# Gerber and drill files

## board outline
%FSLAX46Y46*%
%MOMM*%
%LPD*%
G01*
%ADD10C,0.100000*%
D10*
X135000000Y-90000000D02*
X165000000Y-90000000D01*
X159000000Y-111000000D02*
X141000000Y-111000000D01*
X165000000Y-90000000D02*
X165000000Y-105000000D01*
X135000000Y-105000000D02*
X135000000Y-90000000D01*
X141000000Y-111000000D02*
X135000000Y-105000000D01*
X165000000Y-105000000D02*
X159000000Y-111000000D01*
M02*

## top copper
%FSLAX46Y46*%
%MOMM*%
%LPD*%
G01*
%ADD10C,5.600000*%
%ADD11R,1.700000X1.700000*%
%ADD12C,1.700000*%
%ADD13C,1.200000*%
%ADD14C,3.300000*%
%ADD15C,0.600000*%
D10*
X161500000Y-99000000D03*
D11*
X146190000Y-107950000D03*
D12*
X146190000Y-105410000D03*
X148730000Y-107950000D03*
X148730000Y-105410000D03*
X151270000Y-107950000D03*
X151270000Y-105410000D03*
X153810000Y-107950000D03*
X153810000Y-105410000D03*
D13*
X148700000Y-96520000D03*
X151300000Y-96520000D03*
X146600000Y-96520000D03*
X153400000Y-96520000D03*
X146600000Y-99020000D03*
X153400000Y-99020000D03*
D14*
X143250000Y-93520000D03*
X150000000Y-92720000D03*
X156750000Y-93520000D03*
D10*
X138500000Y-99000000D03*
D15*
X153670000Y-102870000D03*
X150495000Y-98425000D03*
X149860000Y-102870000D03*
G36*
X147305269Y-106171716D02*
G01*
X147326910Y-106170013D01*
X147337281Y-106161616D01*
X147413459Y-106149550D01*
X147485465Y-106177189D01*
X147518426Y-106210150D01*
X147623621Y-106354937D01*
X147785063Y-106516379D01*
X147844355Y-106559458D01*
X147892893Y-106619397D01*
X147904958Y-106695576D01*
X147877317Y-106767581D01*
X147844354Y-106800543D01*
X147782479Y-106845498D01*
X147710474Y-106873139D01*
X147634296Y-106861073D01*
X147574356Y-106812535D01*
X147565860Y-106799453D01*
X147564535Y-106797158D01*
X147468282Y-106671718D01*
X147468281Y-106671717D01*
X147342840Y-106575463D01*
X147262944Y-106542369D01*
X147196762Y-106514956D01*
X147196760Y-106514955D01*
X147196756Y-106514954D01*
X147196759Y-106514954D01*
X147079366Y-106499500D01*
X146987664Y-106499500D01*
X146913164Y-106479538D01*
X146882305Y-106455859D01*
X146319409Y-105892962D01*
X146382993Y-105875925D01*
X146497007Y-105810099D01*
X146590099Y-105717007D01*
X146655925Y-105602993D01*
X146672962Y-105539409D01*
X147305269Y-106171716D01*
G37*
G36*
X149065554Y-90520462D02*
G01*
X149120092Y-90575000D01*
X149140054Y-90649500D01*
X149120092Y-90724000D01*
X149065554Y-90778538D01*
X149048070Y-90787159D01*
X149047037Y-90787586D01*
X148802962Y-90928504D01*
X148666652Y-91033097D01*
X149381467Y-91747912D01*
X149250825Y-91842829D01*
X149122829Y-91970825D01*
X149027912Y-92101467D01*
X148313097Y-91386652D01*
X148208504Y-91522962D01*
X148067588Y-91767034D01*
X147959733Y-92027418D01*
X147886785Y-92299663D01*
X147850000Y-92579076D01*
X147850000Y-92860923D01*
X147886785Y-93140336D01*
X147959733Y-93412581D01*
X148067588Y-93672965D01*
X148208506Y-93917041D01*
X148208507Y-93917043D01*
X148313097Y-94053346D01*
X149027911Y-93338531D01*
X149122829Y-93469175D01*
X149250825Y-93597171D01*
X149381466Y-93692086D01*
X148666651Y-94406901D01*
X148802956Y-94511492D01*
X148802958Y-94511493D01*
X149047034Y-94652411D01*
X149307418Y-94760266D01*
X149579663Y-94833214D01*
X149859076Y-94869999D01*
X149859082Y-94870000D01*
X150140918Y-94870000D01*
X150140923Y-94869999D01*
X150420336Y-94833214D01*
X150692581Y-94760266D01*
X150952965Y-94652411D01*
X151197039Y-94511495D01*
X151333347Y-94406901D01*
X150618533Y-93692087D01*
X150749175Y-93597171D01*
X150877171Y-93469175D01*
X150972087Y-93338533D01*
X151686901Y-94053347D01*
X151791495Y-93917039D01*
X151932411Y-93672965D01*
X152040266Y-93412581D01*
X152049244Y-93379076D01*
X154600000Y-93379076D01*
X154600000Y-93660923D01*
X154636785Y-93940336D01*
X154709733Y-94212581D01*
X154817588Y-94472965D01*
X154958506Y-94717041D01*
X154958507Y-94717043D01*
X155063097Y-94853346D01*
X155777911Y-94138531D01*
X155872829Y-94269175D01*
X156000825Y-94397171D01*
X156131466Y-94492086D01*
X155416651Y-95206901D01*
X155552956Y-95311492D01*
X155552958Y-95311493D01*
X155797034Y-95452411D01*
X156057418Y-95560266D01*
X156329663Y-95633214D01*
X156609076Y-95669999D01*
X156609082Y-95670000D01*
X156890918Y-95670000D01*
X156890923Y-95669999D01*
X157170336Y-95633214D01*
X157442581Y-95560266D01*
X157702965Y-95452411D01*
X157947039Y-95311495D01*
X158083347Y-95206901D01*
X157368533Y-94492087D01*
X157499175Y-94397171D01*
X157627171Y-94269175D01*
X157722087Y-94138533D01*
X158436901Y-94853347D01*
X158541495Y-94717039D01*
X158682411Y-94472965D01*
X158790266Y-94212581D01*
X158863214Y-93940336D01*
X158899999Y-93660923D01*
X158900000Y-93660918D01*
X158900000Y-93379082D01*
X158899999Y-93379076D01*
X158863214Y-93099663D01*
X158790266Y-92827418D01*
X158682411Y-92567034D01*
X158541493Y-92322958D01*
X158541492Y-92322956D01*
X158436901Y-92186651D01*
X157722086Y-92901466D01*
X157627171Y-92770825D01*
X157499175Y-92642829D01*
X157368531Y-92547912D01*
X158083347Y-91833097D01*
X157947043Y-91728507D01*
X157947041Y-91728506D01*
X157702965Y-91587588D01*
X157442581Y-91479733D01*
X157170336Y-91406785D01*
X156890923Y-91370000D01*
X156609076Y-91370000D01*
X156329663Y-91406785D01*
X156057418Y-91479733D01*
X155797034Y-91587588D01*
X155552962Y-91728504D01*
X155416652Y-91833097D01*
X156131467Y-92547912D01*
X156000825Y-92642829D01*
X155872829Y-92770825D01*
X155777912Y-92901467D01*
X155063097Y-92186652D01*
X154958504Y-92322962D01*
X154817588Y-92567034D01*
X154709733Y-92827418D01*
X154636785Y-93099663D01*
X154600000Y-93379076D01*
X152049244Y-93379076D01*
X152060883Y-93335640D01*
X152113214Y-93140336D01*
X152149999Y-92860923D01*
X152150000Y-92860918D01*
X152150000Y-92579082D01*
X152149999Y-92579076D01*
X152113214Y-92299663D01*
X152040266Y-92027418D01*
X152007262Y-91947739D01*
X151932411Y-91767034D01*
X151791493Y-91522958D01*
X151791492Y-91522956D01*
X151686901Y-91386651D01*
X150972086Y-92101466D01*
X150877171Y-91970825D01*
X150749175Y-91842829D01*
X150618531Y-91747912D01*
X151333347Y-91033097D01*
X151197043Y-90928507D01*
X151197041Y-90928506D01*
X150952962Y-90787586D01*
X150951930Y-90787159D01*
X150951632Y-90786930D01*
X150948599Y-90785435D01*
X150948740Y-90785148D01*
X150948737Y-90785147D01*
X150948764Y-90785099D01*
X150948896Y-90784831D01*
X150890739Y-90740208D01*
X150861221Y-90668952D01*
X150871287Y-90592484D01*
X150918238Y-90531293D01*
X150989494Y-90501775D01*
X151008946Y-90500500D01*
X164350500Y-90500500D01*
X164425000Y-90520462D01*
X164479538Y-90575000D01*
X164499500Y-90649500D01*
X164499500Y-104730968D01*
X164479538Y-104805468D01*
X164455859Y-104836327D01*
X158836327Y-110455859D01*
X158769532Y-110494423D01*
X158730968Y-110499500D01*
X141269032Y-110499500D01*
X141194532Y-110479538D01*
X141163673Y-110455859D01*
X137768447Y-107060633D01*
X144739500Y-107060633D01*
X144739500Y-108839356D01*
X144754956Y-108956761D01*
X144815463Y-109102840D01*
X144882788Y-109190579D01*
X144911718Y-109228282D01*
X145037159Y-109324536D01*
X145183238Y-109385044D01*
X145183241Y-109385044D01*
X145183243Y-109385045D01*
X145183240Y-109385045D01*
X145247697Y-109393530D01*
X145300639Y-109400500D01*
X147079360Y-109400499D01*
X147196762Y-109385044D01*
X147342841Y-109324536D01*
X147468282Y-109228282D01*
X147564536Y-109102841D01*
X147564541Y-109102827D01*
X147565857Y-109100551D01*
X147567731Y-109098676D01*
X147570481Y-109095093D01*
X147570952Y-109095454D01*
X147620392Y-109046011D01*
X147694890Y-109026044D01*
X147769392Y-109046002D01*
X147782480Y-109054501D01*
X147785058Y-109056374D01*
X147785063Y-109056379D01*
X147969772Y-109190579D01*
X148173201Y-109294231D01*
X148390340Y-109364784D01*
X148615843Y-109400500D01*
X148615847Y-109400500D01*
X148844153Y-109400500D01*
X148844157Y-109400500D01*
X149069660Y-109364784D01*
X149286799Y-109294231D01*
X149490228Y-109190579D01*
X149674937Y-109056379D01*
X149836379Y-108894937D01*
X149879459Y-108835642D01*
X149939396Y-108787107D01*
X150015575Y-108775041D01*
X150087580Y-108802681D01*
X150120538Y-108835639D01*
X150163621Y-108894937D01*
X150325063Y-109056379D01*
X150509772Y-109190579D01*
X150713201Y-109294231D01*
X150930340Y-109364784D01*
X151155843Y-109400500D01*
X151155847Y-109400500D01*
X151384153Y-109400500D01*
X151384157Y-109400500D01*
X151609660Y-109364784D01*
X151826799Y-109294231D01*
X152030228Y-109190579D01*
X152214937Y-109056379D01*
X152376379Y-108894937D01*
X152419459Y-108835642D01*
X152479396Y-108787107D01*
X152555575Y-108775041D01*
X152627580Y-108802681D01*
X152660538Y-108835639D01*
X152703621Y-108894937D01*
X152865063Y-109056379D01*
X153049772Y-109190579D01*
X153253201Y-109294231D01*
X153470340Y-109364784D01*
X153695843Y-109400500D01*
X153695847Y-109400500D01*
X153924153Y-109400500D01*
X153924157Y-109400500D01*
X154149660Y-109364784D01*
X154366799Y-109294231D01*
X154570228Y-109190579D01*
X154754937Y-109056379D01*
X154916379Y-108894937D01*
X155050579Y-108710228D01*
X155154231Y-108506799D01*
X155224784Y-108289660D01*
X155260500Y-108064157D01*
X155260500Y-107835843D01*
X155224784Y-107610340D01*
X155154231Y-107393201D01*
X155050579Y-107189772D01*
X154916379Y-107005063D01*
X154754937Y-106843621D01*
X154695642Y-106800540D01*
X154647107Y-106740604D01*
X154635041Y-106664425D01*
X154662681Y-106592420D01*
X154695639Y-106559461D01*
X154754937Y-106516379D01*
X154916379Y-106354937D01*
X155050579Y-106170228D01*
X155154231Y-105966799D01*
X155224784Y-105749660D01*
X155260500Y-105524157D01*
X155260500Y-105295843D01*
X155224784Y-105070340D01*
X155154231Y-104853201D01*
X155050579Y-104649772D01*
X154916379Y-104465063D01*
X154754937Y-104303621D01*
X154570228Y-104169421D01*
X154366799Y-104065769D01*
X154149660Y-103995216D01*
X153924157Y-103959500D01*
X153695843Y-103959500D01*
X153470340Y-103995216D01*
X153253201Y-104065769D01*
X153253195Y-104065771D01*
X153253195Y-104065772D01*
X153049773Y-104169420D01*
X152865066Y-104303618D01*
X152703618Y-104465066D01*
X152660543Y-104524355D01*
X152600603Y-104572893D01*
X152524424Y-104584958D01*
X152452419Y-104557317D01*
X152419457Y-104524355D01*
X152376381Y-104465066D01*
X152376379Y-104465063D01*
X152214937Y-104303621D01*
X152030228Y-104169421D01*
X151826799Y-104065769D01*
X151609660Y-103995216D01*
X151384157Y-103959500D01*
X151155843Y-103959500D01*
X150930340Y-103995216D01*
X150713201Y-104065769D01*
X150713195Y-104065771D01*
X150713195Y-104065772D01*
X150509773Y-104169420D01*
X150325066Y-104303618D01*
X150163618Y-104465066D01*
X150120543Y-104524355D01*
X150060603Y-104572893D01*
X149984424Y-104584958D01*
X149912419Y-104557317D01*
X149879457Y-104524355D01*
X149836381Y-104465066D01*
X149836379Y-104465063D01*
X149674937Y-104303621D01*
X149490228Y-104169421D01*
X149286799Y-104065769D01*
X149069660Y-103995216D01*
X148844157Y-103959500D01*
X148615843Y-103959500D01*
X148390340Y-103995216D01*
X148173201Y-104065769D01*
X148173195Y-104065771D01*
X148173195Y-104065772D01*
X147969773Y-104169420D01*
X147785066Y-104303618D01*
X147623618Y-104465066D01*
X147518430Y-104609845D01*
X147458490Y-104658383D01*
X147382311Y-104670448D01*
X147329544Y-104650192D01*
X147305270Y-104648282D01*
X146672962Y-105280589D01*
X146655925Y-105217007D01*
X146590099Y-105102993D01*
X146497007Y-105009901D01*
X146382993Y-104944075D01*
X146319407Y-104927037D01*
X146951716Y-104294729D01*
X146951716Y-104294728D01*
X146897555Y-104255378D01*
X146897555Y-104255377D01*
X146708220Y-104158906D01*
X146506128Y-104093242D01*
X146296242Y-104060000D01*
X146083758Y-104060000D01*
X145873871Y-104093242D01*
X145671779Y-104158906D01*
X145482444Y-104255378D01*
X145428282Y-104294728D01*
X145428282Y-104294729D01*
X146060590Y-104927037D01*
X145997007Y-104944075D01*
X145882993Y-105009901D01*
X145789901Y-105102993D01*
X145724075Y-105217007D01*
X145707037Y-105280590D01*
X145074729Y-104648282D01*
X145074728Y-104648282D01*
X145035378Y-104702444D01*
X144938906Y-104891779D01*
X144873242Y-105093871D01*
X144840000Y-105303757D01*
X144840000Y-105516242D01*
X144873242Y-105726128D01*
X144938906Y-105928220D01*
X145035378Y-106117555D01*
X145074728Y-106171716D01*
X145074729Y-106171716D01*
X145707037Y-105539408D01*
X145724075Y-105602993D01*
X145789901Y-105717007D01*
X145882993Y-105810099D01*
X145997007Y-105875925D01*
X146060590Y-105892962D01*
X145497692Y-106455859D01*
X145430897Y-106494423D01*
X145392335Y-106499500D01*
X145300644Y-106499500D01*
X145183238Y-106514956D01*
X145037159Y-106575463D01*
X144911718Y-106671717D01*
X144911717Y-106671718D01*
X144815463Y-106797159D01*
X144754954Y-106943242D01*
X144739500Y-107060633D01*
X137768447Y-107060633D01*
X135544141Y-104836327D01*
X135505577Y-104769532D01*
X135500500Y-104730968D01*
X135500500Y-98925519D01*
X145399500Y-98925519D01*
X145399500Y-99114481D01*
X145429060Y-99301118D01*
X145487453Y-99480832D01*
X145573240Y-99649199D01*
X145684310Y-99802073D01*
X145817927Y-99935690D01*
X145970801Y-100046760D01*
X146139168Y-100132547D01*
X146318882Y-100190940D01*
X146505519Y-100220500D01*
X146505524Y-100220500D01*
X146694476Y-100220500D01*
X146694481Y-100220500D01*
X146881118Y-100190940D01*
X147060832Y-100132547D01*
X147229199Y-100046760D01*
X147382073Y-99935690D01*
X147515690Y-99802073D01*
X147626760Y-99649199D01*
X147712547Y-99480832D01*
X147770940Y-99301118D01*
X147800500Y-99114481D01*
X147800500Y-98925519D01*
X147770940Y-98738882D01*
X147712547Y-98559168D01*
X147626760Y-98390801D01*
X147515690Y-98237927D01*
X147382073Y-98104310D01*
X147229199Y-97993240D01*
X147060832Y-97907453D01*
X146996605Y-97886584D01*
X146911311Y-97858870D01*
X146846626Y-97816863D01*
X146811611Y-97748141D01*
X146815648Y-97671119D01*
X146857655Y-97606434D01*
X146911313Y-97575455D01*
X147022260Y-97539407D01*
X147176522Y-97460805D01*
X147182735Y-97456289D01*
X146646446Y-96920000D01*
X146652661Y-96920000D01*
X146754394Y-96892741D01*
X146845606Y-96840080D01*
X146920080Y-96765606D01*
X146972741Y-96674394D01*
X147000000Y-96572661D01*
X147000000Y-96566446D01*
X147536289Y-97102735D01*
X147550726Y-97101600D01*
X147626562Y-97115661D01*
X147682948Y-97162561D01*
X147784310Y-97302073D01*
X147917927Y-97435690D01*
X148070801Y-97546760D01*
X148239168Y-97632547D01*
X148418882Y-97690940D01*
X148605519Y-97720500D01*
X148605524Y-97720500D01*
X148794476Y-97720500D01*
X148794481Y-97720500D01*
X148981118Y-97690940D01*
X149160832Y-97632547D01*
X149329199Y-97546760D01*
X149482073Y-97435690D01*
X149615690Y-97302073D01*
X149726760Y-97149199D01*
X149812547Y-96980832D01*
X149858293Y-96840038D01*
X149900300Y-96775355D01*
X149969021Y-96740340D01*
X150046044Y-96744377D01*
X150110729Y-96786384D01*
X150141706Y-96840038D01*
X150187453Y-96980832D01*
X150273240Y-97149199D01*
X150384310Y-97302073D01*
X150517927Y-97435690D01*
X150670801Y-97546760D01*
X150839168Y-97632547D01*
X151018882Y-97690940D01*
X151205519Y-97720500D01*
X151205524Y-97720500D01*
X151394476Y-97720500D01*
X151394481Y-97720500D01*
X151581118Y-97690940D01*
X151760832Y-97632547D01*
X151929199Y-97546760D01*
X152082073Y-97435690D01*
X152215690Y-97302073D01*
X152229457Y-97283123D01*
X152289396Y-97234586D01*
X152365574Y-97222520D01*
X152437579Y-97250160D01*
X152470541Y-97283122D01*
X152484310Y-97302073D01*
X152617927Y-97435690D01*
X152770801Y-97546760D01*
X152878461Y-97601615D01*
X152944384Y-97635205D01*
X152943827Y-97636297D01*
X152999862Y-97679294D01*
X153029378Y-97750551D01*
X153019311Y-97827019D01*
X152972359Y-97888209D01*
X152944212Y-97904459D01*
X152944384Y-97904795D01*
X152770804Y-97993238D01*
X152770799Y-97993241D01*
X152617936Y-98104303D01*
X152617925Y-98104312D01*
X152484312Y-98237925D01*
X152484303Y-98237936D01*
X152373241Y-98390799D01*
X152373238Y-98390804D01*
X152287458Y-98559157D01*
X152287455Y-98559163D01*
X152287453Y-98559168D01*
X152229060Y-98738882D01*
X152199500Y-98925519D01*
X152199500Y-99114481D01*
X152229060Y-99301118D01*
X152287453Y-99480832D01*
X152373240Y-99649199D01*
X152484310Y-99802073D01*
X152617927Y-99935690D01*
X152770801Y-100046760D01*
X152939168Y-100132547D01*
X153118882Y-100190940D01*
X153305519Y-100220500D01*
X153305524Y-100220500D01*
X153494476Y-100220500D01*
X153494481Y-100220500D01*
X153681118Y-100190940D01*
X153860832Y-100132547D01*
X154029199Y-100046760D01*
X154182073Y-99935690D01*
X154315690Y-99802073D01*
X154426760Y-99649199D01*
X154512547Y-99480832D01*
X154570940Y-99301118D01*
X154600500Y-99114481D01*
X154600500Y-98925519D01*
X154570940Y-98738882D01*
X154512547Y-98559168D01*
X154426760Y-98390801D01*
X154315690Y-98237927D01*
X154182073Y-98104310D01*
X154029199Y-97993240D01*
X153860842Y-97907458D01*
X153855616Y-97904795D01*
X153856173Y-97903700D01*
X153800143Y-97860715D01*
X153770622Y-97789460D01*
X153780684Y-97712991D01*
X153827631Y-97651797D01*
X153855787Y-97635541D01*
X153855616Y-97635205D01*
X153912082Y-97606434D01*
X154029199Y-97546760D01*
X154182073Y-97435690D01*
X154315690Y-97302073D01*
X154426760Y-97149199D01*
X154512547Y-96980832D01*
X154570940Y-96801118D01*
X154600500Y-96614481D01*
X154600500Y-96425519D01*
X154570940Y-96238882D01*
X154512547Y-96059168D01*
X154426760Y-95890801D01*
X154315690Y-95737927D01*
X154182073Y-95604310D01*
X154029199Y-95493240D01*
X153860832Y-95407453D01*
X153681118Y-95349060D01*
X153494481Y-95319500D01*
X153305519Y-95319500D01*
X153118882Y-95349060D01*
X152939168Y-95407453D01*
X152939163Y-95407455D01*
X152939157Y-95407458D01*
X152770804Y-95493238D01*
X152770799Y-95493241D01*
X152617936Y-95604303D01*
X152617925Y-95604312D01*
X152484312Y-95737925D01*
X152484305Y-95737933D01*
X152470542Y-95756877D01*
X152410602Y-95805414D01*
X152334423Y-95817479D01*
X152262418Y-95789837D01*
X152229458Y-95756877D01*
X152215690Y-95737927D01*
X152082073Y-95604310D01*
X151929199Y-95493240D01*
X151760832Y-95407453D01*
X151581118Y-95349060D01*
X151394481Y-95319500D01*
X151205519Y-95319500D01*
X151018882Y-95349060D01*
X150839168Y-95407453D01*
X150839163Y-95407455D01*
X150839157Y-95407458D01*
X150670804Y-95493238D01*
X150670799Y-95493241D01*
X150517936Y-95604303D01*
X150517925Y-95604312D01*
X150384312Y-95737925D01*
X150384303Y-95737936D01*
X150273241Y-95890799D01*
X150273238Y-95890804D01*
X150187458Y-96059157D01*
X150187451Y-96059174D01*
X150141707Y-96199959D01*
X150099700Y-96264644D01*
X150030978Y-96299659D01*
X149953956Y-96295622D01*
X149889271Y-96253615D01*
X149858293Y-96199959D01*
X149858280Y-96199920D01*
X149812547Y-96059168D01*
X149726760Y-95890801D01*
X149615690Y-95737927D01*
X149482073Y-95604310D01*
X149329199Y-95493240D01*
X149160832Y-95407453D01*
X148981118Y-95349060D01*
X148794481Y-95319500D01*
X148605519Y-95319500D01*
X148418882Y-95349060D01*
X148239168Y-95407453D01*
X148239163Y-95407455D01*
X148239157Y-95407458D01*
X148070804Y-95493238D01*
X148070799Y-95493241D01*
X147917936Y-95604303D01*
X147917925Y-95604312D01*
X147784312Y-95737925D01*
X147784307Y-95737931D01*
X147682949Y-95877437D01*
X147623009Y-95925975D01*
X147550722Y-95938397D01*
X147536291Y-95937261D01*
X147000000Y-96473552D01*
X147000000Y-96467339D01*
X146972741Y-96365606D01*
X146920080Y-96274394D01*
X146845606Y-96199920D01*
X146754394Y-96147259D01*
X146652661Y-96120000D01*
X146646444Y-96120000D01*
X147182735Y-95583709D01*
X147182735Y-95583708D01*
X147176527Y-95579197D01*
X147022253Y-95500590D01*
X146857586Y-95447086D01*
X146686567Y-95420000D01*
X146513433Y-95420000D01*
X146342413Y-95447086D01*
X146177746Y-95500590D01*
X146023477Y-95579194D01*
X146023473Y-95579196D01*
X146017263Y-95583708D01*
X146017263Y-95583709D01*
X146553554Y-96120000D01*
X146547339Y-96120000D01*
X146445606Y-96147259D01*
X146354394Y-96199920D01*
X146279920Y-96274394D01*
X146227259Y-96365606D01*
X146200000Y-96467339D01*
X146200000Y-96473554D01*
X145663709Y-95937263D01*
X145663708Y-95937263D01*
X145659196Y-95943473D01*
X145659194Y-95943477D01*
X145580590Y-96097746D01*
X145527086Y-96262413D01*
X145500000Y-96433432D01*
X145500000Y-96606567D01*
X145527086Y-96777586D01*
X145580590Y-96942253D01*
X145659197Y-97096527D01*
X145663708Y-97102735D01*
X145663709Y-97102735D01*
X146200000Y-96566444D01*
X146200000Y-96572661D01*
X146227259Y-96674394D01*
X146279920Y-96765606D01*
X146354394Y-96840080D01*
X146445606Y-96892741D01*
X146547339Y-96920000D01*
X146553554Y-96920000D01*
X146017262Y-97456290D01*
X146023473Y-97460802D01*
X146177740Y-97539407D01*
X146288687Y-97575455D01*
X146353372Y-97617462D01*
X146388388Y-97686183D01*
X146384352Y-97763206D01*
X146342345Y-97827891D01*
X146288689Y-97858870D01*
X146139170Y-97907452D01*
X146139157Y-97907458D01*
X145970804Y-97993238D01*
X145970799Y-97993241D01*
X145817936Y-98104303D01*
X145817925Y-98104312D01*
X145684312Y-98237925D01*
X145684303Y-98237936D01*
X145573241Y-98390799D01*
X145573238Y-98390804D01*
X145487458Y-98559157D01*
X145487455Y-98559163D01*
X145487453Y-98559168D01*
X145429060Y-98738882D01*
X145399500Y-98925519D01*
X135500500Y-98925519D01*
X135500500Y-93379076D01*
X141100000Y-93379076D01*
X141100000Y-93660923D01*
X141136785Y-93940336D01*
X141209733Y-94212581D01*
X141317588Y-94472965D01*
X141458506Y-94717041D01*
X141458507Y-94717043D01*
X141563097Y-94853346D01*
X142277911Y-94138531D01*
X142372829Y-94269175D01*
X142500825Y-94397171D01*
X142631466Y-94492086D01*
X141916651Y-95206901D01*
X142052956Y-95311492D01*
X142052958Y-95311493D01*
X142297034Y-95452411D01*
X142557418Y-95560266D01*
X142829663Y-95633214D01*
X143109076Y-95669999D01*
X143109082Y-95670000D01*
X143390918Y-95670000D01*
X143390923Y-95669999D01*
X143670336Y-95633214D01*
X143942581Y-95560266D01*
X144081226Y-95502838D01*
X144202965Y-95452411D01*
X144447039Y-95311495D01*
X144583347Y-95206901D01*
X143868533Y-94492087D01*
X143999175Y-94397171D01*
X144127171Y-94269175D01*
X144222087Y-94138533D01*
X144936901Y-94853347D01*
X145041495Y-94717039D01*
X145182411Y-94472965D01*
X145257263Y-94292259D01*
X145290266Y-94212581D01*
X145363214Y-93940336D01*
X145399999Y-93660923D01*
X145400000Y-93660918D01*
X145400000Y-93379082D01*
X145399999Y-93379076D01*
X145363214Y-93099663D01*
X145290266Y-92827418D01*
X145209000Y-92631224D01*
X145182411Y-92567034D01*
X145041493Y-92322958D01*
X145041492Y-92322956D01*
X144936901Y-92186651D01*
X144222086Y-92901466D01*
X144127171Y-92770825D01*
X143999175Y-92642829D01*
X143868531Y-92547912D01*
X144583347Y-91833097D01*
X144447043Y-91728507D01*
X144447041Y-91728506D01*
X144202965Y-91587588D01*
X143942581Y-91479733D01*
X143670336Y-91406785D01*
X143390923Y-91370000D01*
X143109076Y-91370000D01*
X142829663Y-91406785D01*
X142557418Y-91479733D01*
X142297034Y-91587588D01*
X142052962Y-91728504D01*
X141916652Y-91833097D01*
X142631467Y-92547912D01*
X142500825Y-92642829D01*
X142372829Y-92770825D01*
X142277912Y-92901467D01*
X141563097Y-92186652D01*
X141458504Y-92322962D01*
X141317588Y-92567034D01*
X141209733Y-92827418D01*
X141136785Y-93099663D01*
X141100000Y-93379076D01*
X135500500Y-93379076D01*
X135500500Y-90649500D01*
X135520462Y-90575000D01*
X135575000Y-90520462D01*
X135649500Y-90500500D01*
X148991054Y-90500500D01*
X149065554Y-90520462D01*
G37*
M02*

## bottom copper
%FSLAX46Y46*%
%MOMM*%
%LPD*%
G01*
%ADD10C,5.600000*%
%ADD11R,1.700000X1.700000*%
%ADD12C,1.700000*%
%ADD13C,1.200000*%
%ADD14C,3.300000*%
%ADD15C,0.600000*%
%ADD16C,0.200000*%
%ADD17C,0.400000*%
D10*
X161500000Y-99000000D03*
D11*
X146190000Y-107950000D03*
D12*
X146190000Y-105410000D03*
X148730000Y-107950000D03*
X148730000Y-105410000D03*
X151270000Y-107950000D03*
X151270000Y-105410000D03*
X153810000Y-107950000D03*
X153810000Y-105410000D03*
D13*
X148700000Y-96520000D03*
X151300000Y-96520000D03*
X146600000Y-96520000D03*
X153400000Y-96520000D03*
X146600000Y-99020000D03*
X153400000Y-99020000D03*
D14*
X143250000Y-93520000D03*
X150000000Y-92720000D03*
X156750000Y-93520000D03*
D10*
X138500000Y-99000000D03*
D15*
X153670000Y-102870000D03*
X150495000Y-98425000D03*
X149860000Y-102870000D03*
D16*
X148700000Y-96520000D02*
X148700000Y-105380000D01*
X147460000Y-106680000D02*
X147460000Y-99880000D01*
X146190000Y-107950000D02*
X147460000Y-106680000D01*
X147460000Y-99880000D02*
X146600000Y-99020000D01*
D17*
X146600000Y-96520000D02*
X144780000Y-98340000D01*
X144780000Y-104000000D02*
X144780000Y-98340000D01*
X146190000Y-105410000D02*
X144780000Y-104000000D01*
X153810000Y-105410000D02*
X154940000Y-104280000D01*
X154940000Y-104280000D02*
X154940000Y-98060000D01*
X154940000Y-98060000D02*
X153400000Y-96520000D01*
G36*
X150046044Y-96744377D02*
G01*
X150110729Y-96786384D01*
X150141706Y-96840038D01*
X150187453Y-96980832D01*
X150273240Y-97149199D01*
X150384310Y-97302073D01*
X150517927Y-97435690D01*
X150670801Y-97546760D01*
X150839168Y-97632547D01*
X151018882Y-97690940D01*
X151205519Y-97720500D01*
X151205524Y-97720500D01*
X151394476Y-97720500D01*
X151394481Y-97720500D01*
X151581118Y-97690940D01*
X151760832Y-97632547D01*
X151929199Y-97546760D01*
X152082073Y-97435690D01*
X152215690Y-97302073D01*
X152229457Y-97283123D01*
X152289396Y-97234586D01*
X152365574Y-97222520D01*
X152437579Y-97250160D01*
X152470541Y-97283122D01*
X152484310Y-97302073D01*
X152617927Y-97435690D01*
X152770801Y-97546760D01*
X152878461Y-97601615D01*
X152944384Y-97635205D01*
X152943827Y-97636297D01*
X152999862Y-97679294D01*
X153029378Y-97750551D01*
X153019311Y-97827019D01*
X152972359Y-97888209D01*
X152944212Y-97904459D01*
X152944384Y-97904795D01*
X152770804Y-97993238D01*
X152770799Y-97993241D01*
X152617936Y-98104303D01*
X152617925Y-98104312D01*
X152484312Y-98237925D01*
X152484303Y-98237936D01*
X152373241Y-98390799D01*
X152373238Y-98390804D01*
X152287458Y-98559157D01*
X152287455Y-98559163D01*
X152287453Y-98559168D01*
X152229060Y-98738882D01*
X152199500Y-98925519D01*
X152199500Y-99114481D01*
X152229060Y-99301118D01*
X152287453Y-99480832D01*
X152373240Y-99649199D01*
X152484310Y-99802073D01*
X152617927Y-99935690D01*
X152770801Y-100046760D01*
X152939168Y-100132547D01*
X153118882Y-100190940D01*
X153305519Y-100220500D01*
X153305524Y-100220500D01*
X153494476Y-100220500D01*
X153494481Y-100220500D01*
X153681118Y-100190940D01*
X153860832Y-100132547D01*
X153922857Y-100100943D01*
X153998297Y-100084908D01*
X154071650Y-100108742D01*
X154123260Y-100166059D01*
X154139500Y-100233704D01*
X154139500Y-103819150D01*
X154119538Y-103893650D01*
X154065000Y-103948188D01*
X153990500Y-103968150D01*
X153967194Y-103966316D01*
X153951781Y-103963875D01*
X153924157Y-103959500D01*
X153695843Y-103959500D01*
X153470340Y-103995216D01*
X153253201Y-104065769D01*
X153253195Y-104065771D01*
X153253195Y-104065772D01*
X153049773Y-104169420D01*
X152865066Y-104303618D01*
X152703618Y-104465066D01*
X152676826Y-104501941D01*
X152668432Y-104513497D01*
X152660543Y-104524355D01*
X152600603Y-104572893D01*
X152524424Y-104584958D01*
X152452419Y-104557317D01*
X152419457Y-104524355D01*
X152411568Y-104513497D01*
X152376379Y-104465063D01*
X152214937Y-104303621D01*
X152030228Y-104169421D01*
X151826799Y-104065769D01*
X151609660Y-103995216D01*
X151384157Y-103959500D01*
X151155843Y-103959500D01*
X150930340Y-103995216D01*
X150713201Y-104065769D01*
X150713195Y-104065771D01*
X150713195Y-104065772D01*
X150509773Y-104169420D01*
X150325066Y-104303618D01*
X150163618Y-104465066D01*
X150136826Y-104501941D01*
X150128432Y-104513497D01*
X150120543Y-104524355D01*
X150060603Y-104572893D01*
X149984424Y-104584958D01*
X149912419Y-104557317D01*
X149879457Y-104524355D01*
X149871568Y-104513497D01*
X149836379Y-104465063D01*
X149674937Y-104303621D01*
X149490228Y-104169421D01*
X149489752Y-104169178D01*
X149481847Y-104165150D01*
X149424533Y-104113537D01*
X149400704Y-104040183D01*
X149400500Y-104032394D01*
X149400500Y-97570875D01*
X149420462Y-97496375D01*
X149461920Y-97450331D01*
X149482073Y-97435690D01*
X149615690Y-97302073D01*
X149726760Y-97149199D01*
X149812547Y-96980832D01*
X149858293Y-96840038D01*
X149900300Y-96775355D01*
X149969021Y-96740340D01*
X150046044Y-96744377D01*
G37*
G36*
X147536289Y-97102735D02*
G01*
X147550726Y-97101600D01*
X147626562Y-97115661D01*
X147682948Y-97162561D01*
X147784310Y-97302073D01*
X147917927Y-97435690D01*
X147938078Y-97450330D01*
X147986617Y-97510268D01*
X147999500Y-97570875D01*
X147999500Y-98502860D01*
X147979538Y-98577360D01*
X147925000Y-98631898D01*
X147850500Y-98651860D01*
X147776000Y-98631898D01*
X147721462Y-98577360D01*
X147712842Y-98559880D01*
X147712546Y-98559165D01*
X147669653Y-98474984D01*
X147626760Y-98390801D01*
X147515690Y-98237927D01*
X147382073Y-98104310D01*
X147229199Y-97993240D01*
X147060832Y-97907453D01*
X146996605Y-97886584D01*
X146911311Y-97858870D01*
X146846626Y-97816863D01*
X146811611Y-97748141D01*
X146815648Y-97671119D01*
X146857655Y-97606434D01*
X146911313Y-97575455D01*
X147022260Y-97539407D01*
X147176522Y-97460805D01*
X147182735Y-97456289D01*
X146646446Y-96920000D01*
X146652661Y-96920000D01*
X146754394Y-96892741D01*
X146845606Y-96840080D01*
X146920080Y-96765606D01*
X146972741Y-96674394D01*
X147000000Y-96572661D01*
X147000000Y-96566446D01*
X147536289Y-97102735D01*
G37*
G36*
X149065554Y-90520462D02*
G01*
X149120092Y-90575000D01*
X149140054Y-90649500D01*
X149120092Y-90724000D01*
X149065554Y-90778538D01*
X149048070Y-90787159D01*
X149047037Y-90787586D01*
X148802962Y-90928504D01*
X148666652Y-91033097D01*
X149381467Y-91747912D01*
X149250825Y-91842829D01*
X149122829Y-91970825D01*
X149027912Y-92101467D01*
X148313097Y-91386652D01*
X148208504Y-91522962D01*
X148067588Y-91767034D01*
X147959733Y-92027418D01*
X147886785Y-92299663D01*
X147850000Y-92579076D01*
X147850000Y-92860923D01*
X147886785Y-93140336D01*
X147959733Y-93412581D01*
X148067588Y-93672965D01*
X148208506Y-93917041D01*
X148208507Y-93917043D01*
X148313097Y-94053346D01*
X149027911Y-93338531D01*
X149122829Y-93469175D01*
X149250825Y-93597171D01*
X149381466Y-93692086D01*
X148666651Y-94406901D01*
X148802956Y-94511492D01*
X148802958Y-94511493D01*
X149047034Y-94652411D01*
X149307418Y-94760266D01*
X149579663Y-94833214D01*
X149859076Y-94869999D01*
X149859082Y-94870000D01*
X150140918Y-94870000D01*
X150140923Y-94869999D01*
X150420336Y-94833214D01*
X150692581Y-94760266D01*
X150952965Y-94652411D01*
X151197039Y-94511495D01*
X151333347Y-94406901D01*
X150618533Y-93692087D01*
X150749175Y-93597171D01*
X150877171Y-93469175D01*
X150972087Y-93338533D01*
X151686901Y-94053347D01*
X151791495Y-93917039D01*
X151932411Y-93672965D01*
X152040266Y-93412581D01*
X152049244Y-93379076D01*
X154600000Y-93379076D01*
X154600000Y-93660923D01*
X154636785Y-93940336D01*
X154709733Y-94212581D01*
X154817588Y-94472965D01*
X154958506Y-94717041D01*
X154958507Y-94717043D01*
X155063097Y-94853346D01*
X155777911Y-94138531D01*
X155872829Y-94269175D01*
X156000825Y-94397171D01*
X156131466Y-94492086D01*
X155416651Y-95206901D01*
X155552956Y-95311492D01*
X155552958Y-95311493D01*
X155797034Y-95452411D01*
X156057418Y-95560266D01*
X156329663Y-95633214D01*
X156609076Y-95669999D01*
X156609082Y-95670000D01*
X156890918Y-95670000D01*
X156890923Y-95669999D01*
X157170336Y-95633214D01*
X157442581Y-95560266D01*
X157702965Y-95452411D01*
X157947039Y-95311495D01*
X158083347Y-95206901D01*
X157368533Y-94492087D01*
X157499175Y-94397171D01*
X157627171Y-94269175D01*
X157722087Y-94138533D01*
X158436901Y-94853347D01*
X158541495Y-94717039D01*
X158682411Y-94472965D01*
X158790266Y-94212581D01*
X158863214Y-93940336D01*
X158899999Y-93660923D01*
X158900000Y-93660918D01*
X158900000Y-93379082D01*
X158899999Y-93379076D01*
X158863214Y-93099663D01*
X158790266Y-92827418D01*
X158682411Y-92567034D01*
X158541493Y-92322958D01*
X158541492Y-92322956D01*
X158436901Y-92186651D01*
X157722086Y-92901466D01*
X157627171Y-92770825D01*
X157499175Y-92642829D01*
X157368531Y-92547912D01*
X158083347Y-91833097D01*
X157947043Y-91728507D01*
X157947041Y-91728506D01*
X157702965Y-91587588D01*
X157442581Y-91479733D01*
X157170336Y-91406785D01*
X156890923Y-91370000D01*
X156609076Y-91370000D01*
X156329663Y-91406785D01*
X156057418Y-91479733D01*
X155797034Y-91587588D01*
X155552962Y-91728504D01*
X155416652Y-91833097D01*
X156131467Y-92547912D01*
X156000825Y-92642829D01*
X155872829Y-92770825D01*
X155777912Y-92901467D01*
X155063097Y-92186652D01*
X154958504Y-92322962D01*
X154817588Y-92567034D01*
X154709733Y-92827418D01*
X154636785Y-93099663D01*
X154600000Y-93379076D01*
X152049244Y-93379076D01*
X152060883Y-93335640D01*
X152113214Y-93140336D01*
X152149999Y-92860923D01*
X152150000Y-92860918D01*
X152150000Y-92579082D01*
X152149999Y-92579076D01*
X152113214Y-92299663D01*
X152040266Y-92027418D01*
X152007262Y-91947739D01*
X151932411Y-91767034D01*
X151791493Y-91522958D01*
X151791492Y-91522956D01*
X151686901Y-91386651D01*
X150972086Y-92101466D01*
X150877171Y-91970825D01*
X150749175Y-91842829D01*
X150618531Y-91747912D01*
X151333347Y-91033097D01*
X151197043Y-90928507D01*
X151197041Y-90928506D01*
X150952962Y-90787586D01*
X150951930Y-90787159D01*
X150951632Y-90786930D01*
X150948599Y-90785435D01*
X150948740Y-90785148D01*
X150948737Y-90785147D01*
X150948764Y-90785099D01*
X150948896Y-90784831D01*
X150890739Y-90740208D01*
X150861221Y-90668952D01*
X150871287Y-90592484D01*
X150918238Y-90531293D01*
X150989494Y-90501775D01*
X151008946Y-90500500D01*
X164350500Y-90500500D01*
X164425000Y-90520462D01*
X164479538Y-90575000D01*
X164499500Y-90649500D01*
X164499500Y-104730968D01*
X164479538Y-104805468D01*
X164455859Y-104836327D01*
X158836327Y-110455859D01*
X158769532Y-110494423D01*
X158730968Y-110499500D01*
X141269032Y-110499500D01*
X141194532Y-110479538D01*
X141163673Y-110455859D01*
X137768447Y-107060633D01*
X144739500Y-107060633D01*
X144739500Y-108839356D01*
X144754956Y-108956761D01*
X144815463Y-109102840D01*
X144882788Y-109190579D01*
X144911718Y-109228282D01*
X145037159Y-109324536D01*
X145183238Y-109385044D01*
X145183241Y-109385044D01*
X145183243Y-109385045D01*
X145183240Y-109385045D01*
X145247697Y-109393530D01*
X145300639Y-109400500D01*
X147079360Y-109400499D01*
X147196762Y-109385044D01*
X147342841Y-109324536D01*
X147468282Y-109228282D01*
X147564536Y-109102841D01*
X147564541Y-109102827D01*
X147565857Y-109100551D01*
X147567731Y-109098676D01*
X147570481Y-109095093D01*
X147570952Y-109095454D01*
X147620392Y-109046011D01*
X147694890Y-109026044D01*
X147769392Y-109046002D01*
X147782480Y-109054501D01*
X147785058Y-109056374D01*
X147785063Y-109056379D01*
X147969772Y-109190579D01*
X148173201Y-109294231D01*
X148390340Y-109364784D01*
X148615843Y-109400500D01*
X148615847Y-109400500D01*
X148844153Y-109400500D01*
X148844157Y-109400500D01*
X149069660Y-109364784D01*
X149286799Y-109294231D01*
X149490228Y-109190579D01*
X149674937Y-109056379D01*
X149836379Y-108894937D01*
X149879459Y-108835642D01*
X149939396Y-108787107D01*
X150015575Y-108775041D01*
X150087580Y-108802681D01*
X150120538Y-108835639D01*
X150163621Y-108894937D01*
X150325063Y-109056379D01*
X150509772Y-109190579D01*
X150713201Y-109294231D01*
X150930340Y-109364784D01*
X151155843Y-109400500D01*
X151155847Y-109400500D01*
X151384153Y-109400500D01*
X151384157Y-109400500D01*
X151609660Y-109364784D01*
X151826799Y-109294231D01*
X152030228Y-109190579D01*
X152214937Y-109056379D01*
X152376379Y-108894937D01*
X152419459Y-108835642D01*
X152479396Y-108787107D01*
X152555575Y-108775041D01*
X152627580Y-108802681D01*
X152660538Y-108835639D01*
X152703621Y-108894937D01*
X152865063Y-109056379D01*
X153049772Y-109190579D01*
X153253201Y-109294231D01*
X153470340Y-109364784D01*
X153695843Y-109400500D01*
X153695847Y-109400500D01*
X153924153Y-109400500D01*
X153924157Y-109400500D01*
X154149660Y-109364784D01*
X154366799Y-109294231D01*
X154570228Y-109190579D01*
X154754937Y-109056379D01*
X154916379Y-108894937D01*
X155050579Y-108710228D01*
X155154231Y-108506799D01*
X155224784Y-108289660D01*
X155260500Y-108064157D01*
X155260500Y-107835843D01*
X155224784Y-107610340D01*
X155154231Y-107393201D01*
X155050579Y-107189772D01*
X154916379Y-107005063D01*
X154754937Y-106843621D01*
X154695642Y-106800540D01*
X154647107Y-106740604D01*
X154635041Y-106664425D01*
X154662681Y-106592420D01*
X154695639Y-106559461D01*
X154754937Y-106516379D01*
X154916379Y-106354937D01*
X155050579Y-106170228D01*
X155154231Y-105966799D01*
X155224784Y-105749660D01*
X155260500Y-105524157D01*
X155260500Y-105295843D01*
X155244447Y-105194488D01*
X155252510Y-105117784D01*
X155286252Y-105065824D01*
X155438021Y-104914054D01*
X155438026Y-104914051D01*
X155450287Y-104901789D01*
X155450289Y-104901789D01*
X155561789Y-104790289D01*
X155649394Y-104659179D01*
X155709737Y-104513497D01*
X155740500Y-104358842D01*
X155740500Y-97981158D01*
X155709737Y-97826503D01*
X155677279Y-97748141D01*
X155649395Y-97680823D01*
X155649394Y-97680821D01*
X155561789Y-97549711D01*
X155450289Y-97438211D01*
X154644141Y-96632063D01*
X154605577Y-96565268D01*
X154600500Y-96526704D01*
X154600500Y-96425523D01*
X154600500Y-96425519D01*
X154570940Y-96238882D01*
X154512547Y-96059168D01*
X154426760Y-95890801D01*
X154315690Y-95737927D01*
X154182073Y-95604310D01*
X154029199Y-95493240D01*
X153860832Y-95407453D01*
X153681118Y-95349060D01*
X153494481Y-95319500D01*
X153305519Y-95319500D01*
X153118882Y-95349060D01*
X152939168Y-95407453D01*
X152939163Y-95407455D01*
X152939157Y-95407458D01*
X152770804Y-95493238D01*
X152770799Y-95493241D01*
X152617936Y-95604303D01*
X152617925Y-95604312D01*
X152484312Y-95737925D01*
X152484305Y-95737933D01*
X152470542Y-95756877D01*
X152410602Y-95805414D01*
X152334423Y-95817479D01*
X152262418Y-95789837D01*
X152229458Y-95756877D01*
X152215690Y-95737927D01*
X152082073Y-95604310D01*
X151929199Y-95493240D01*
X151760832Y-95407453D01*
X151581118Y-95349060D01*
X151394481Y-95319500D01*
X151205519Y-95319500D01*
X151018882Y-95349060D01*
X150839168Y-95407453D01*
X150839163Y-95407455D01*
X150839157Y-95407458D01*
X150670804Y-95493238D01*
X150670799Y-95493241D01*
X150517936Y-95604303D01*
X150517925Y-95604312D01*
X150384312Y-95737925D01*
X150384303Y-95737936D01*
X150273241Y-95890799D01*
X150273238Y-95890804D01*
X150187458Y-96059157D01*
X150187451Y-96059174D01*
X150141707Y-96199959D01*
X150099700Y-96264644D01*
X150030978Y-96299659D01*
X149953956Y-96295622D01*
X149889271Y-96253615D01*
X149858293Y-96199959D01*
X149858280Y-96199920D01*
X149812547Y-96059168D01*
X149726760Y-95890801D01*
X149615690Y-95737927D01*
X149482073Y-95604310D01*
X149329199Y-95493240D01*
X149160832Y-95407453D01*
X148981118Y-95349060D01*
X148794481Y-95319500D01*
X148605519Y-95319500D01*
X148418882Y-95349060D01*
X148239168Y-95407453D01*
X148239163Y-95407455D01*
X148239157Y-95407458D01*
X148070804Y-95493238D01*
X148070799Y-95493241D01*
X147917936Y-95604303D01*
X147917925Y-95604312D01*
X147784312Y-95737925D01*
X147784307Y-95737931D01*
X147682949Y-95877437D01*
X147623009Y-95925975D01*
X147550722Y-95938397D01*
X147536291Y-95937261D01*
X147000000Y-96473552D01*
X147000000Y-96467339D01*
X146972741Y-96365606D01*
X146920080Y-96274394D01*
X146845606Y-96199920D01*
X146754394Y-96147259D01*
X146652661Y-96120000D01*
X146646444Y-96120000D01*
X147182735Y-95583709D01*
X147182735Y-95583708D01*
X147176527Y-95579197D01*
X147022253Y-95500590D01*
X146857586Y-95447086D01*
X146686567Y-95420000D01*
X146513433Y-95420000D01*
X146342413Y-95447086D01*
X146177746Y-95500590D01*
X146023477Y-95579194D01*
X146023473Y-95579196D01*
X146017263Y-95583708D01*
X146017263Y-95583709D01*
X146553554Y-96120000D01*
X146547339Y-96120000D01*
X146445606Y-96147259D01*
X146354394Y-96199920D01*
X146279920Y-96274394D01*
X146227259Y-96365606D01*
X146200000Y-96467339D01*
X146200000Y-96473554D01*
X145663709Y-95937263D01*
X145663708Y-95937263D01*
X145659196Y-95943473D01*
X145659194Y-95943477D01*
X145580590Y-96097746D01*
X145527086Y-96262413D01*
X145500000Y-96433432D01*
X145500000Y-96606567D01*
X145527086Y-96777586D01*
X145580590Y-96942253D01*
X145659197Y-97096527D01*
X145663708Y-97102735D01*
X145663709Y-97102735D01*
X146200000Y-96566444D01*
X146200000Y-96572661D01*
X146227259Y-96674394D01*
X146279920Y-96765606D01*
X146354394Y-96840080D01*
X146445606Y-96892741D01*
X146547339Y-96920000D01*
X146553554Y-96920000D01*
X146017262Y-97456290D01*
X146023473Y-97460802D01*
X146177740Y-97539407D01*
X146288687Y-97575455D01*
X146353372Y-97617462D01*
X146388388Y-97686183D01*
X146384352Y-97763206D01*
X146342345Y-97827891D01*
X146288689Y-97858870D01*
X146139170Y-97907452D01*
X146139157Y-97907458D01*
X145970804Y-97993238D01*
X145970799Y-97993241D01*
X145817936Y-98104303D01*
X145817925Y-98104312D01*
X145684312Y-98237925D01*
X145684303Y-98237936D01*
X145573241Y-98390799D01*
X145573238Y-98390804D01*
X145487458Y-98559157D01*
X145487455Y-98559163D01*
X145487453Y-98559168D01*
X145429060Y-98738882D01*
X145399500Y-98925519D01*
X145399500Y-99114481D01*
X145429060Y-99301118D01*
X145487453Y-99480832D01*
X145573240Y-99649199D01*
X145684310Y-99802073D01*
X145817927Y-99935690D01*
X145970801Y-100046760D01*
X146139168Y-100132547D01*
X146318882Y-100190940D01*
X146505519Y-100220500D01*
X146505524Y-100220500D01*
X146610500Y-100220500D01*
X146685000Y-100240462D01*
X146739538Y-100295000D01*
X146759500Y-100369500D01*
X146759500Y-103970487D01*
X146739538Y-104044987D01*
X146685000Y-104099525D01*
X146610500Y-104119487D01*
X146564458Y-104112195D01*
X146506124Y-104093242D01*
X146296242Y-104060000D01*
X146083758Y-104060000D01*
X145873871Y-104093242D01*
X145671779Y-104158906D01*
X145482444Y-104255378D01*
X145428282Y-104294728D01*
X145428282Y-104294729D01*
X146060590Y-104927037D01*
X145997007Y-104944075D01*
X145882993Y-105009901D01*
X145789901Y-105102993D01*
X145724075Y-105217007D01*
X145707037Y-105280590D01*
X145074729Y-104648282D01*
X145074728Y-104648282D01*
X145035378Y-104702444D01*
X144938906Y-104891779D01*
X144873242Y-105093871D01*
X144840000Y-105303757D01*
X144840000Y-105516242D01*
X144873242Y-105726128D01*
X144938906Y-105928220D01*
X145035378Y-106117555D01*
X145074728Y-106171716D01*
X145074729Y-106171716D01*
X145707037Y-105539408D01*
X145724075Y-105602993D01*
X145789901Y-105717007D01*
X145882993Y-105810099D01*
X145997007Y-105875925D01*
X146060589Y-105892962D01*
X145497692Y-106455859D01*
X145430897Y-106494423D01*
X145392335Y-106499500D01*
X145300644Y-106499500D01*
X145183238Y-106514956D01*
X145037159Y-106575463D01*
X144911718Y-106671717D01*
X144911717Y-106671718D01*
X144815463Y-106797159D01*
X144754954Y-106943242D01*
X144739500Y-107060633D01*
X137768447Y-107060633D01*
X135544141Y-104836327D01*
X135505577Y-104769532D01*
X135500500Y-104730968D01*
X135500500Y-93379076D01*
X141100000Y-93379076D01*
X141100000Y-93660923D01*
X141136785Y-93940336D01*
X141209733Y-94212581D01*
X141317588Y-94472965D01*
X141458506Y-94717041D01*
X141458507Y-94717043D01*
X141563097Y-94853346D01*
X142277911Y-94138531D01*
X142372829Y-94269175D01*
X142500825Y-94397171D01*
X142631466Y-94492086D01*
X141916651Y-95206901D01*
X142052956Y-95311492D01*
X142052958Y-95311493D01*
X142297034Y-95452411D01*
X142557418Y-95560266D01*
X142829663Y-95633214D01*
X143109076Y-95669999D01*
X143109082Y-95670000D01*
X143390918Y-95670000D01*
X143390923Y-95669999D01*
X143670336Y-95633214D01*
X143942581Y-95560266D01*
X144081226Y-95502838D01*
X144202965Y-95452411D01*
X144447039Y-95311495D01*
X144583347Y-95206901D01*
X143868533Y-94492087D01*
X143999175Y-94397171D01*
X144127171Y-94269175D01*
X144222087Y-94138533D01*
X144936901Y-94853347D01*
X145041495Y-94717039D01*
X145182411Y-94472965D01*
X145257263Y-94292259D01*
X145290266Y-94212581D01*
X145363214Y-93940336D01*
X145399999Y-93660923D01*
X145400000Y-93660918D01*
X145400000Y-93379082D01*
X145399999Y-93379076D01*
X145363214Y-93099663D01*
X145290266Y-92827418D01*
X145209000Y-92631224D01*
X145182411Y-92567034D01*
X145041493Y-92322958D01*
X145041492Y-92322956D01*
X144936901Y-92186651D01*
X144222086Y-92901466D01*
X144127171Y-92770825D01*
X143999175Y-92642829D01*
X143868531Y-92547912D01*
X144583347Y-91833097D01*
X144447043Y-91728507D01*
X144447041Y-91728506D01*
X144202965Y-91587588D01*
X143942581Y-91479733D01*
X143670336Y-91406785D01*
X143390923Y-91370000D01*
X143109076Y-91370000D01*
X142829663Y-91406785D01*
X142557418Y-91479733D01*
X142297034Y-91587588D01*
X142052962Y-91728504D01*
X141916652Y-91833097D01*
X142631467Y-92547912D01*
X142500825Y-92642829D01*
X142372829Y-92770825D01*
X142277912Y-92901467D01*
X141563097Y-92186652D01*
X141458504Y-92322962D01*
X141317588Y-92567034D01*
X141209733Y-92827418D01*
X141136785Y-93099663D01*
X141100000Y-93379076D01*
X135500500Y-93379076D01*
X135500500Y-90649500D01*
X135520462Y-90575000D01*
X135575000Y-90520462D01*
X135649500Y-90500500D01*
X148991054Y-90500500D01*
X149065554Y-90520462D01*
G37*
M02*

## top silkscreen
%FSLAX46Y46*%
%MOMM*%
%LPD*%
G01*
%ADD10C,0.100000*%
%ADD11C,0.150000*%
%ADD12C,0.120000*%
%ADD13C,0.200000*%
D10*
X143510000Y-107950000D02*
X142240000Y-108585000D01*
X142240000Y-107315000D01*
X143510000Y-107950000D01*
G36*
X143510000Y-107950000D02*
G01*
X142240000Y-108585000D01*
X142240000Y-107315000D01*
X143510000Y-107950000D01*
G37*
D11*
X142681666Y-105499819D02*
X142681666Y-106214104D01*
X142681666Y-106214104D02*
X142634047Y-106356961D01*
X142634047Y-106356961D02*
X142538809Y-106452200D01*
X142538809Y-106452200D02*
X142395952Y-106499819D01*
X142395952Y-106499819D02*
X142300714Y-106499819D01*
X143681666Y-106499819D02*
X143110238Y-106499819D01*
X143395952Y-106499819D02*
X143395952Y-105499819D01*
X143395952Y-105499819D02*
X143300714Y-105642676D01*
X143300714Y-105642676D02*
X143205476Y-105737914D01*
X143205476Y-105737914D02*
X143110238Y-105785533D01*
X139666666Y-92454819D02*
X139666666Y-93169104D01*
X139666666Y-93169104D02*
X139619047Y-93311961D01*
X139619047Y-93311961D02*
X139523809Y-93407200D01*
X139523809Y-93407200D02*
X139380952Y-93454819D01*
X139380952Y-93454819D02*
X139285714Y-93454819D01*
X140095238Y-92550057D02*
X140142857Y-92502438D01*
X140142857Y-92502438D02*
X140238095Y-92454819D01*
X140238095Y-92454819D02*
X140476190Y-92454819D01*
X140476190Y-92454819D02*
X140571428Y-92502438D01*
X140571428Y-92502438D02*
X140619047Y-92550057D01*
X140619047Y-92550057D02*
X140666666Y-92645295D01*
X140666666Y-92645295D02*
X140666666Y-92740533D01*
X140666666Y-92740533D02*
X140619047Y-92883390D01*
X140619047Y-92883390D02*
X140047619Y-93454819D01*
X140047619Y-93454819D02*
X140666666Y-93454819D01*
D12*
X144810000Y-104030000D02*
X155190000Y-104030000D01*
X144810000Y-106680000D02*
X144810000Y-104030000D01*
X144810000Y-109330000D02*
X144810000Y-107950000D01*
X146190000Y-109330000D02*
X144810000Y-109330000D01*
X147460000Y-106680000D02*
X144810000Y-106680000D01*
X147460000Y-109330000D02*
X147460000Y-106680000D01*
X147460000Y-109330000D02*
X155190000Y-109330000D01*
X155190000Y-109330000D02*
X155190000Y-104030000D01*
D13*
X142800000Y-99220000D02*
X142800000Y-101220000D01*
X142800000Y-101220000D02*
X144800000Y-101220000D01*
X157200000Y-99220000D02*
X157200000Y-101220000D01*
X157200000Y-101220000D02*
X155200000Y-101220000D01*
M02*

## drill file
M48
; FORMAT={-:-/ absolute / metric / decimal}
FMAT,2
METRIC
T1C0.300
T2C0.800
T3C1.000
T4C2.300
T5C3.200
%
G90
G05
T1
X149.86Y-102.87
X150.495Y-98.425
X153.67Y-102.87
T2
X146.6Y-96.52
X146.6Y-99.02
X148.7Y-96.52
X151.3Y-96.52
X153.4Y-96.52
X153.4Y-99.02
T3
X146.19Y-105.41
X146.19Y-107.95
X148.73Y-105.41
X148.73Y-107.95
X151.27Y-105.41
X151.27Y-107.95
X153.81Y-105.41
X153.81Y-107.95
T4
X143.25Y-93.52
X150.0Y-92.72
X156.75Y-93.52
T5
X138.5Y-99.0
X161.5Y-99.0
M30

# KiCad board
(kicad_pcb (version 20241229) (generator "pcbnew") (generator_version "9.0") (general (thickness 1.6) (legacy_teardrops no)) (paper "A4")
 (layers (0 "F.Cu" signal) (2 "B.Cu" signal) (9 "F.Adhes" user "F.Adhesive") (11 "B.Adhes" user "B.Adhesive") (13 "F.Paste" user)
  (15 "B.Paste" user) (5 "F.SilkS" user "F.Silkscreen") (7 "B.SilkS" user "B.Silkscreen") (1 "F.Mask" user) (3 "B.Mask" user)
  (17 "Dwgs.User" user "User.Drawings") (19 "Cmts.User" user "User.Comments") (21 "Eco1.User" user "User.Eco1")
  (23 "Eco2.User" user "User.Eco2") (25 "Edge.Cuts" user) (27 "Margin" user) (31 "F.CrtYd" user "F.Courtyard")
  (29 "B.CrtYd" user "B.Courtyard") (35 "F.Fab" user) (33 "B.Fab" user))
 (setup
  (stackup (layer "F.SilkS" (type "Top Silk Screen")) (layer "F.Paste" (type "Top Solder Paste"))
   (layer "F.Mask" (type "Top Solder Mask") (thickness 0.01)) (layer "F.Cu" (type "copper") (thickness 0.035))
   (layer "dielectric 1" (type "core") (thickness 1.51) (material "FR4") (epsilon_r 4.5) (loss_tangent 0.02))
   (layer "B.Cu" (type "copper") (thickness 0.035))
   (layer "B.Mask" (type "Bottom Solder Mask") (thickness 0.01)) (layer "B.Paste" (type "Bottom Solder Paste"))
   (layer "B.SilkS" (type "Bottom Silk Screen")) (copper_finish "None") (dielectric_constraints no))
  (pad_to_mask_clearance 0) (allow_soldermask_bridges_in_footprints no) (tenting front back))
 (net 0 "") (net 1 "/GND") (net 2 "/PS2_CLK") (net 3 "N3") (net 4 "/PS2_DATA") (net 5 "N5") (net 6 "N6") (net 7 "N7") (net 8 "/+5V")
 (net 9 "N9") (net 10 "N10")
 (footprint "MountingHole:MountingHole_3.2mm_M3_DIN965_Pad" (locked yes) (layer "F.Cu") (at 161.5 99)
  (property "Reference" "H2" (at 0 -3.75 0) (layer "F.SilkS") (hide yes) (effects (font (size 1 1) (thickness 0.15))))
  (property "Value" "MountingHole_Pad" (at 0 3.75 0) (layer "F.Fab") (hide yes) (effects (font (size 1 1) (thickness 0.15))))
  (pad "1" thru_hole circle (at 0 0) (size 5.6 5.6) (drill 3.2) (layers "*.Cu" "*.Mask") (remove_unused_layers no) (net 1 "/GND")
   (zone_connect 2)))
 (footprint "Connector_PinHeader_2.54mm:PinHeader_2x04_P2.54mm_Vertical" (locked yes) (layer "F.Cu") (at 146.19 107.95 90)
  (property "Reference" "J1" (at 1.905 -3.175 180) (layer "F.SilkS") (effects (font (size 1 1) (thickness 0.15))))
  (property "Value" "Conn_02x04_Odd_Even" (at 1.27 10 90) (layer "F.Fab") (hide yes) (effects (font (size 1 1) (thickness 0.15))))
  (fp_line (start 3.92 -1.38) (end 3.92 9) (stroke (width 0.12) (type solid)) (layer "F.SilkS"))
  (fp_line (start 1.27 -1.38) (end 3.92 -1.38) (stroke (width 0.12) (type solid)) (layer "F.SilkS"))
  (fp_line (start -1.38 -1.38) (end 0 -1.38) (stroke (width 0.12) (type solid)) (layer "F.SilkS"))
  (fp_line (start -1.38 0) (end -1.38 -1.38) (stroke (width 0.12) (type solid)) (layer "F.SilkS"))
  (fp_line (start 1.27 1.27) (end 1.27 -1.38) (stroke (width 0.12) (type solid)) (layer "F.SilkS"))
  (fp_line (start -1.38 1.27) (end 1.27 1.27) (stroke (width 0.12) (type solid)) (layer "F.SilkS"))
  (fp_line (start -1.38 1.27) (end -1.38 9) (stroke (width 0.12) (type solid)) (layer "F.SilkS"))
  (fp_line (start -1.38 9) (end 3.92 9) (stroke (width 0.12) (type solid)) (layer "F.SilkS"))
  (pad "1" thru_hole rect (at 0 0 90) (size 1.7 1.7) (drill 1) (layers "*.Cu" "*.Mask") (remove_unused_layers no) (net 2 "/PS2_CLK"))
  (pad "2" thru_hole circle (at 2.54 0 90) (size 1.7 1.7) (drill 1) (layers "*.Cu" "*.Mask") (remove_unused_layers no) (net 1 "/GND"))
  (pad "3" thru_hole circle (at 0 2.54 90) (size 1.7 1.7) (drill 1) (layers "*.Cu" "*.Mask") (remove_unused_layers no) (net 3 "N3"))
  (pad "4" thru_hole circle (at 2.54 2.54 90) (size 1.7 1.7) (drill 1) (layers "*.Cu" "*.Mask") (remove_unused_layers no)
   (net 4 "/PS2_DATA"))
  (pad "5" thru_hole circle (at 0 5.08 90) (size 1.7 1.7) (drill 1) (layers "*.Cu" "*.Mask") (remove_unused_layers no) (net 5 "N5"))
  (pad "6" thru_hole circle (at 2.54 5.08 90) (size 1.7 1.7) (drill 1) (layers "*.Cu" "*.Mask") (remove_unused_layers no) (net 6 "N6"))
  (pad "7" thru_hole circle (at 0 7.62 90) (size 1.7 1.7) (drill 1) (layers "*.Cu" "*.Mask") (remove_unused_layers no) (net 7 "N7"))
  (pad "8" thru_hole circle (at 2.54 7.62 90) (size 1.7 1.7) (drill 1) (layers "*.Cu" "*.Mask") (remove_unused_layers no) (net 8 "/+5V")))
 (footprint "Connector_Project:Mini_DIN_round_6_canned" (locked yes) (layer "F.Cu") (at 150 88.02)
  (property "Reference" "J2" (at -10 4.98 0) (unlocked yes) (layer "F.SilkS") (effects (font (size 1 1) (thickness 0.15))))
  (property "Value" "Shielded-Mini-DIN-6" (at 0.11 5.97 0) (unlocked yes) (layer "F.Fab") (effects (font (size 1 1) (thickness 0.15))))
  (fp_line (start -7.2 11.2) (end -7.2 13.2) (stroke (width 0.2) (type solid)) (layer "F.SilkS"))
  (fp_line (start -7.2 13.2) (end -5.2 13.2) (stroke (width 0.2) (type solid)) (layer "F.SilkS"))
  (fp_line (start 7.2 11.2) (end 7.2 13.2) (stroke (width 0.2) (type solid)) (layer "F.SilkS"))
  (fp_line (start 7.2 13.2) (end 5.2 13.2) (stroke (width 0.2) (type solid)) (layer "F.SilkS"))
  (pad "1" thru_hole circle (at -1.3 8.5 90) (size 1.2 1.2) (drill 0.8) (layers "*.Cu" "*.Mask") (remove_unused_layers no)
   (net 4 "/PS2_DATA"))
  (pad "2" thru_hole circle (at 1.3 8.5 90) (size 1.2 1.2) (drill 0.8) (layers "*.Cu" "*.Mask") (remove_unused_layers no) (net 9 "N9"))
  (pad "3" thru_hole circle (at -3.4 8.5 90) (size 1.2 1.2) (drill 0.8) (layers "*.Cu" "*.Mask") (remove_unused_layers no) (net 1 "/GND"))
  (pad "4" thru_hole circle (at 3.4 8.5 90) (size 1.2 1.2) (drill 0.8) (layers "*.Cu" "*.Mask") (remove_unused_layers no) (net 8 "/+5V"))
  (pad "5" thru_hole circle (at -3.4 11 90) (size 1.2 1.2) (drill 0.8) (layers "*.Cu" "*.Mask") (remove_unused_layers no) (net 2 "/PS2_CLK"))
  (pad "6" thru_hole circle (at 3.4 11 90) (size 1.2 1.2) (drill 0.8) (layers "*.Cu" "*.Mask") (remove_unused_layers no) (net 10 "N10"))
  (pad "SH" thru_hole circle (at -6.75 5.5) (size 3.3 3.3) (drill 2.3) (layers "*.Cu" "*.Mask") (remove_unused_layers no) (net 1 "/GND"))
  (pad "SH" thru_hole circle (at 0 4.7) (size 3.3 3.3) (drill 2.3) (layers "*.Cu" "*.Mask") (remove_unused_layers no) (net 1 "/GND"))
  (pad "SH" thru_hole circle (at 6.75 5.5) (size 3.3 3.3) (drill 2.3) (layers "*.Cu" "*.Mask") (remove_unused_layers no) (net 1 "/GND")))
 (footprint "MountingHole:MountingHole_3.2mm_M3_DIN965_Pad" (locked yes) (layer "F.Cu") (at 138.5 99)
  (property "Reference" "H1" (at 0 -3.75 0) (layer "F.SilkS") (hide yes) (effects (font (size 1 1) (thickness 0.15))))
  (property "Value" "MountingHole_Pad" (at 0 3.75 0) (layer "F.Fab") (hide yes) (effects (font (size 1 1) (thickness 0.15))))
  (pad "1" thru_hole circle (at 0 0) (size 5.6 5.6) (drill 3.2) (layers "*.Cu" "*.Mask") (remove_unused_layers no) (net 1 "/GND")
   (zone_connect 2)))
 (gr_poly (pts (xy 143.51 107.95) (xy 142.24 108.585) (xy 142.24 107.315)) (stroke (width 0.1) (type solid)) (fill yes) (layer "F.SilkS"))
 (gr_line (start 135 90) (end 165 90) (stroke (width 0.1) (type default)) (locked yes) (layer "Edge.Cuts"))
 (gr_line (start 159 111) (end 141 111) (stroke (width 0.1) (type default)) (locked yes) (layer "Edge.Cuts"))
 (gr_line (start 165 90) (end 165 105) (stroke (width 0.1) (type default)) (locked yes) (layer "Edge.Cuts"))
 (gr_line (start 135 105) (end 135 90) (stroke (width 0.1) (type solid)) (locked yes) (layer "Edge.Cuts"))
 (gr_line (start 141 111) (end 135 105) (stroke (width 0.1) (type default)) (locked yes) (layer "Edge.Cuts"))
 (gr_line (start 165 105) (end 159 111) (stroke (width 0.1) (type solid)) (locked yes) (layer "Edge.Cuts"))
 (segment (start 148.7 96.52) (end 148.7 105.38) (width 0.2) (layer "B.Cu") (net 4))
 (segment (start 147.46 106.68) (end 147.46 99.88) (width 0.2) (layer "B.Cu") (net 2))
 (segment (start 146.19 107.95) (end 147.46 106.68) (width 0.2) (layer "B.Cu") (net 2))
 (segment (start 147.46 99.88) (end 146.6 99.02) (width 0.2) (layer "B.Cu") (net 2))
 (via (at 153.67 102.87) (size 0.6) (drill 0.3) (layers "F.Cu" "B.Cu") (free yes) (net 1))
 (via (at 150.495 98.425) (size 0.6) (drill 0.3) (layers "F.Cu" "B.Cu") (free yes) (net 1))
 (via (at 149.86 102.87) (size 0.6) (drill 0.3) (layers "F.Cu" "B.Cu") (free yes) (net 1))
 (segment (start 146.6 96.52) (end 144.78 98.34) (width 0.4) (layer "B.Cu") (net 1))
 (segment (start 144.78 104) (end 144.78 98.34) (width 0.4) (layer "B.Cu") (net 1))
 (segment (start 146.19 105.41) (end 144.78 104) (width 0.4) (layer "B.Cu") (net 1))
 (segment (start 153.81 105.41) (end 154.94 104.28) (width 0.4) (layer "B.Cu") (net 8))
 (segment (start 154.94 104.28) (end 154.94 98.06) (width 0.4) (layer "B.Cu") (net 8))
 (segment (start 154.94 98.06) (end 153.4 96.52) (width 0.4) (layer "B.Cu") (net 8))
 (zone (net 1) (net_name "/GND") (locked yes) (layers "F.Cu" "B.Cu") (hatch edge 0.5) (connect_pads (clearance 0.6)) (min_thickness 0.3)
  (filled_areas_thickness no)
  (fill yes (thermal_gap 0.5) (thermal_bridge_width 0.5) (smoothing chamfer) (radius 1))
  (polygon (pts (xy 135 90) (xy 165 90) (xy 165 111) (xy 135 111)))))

